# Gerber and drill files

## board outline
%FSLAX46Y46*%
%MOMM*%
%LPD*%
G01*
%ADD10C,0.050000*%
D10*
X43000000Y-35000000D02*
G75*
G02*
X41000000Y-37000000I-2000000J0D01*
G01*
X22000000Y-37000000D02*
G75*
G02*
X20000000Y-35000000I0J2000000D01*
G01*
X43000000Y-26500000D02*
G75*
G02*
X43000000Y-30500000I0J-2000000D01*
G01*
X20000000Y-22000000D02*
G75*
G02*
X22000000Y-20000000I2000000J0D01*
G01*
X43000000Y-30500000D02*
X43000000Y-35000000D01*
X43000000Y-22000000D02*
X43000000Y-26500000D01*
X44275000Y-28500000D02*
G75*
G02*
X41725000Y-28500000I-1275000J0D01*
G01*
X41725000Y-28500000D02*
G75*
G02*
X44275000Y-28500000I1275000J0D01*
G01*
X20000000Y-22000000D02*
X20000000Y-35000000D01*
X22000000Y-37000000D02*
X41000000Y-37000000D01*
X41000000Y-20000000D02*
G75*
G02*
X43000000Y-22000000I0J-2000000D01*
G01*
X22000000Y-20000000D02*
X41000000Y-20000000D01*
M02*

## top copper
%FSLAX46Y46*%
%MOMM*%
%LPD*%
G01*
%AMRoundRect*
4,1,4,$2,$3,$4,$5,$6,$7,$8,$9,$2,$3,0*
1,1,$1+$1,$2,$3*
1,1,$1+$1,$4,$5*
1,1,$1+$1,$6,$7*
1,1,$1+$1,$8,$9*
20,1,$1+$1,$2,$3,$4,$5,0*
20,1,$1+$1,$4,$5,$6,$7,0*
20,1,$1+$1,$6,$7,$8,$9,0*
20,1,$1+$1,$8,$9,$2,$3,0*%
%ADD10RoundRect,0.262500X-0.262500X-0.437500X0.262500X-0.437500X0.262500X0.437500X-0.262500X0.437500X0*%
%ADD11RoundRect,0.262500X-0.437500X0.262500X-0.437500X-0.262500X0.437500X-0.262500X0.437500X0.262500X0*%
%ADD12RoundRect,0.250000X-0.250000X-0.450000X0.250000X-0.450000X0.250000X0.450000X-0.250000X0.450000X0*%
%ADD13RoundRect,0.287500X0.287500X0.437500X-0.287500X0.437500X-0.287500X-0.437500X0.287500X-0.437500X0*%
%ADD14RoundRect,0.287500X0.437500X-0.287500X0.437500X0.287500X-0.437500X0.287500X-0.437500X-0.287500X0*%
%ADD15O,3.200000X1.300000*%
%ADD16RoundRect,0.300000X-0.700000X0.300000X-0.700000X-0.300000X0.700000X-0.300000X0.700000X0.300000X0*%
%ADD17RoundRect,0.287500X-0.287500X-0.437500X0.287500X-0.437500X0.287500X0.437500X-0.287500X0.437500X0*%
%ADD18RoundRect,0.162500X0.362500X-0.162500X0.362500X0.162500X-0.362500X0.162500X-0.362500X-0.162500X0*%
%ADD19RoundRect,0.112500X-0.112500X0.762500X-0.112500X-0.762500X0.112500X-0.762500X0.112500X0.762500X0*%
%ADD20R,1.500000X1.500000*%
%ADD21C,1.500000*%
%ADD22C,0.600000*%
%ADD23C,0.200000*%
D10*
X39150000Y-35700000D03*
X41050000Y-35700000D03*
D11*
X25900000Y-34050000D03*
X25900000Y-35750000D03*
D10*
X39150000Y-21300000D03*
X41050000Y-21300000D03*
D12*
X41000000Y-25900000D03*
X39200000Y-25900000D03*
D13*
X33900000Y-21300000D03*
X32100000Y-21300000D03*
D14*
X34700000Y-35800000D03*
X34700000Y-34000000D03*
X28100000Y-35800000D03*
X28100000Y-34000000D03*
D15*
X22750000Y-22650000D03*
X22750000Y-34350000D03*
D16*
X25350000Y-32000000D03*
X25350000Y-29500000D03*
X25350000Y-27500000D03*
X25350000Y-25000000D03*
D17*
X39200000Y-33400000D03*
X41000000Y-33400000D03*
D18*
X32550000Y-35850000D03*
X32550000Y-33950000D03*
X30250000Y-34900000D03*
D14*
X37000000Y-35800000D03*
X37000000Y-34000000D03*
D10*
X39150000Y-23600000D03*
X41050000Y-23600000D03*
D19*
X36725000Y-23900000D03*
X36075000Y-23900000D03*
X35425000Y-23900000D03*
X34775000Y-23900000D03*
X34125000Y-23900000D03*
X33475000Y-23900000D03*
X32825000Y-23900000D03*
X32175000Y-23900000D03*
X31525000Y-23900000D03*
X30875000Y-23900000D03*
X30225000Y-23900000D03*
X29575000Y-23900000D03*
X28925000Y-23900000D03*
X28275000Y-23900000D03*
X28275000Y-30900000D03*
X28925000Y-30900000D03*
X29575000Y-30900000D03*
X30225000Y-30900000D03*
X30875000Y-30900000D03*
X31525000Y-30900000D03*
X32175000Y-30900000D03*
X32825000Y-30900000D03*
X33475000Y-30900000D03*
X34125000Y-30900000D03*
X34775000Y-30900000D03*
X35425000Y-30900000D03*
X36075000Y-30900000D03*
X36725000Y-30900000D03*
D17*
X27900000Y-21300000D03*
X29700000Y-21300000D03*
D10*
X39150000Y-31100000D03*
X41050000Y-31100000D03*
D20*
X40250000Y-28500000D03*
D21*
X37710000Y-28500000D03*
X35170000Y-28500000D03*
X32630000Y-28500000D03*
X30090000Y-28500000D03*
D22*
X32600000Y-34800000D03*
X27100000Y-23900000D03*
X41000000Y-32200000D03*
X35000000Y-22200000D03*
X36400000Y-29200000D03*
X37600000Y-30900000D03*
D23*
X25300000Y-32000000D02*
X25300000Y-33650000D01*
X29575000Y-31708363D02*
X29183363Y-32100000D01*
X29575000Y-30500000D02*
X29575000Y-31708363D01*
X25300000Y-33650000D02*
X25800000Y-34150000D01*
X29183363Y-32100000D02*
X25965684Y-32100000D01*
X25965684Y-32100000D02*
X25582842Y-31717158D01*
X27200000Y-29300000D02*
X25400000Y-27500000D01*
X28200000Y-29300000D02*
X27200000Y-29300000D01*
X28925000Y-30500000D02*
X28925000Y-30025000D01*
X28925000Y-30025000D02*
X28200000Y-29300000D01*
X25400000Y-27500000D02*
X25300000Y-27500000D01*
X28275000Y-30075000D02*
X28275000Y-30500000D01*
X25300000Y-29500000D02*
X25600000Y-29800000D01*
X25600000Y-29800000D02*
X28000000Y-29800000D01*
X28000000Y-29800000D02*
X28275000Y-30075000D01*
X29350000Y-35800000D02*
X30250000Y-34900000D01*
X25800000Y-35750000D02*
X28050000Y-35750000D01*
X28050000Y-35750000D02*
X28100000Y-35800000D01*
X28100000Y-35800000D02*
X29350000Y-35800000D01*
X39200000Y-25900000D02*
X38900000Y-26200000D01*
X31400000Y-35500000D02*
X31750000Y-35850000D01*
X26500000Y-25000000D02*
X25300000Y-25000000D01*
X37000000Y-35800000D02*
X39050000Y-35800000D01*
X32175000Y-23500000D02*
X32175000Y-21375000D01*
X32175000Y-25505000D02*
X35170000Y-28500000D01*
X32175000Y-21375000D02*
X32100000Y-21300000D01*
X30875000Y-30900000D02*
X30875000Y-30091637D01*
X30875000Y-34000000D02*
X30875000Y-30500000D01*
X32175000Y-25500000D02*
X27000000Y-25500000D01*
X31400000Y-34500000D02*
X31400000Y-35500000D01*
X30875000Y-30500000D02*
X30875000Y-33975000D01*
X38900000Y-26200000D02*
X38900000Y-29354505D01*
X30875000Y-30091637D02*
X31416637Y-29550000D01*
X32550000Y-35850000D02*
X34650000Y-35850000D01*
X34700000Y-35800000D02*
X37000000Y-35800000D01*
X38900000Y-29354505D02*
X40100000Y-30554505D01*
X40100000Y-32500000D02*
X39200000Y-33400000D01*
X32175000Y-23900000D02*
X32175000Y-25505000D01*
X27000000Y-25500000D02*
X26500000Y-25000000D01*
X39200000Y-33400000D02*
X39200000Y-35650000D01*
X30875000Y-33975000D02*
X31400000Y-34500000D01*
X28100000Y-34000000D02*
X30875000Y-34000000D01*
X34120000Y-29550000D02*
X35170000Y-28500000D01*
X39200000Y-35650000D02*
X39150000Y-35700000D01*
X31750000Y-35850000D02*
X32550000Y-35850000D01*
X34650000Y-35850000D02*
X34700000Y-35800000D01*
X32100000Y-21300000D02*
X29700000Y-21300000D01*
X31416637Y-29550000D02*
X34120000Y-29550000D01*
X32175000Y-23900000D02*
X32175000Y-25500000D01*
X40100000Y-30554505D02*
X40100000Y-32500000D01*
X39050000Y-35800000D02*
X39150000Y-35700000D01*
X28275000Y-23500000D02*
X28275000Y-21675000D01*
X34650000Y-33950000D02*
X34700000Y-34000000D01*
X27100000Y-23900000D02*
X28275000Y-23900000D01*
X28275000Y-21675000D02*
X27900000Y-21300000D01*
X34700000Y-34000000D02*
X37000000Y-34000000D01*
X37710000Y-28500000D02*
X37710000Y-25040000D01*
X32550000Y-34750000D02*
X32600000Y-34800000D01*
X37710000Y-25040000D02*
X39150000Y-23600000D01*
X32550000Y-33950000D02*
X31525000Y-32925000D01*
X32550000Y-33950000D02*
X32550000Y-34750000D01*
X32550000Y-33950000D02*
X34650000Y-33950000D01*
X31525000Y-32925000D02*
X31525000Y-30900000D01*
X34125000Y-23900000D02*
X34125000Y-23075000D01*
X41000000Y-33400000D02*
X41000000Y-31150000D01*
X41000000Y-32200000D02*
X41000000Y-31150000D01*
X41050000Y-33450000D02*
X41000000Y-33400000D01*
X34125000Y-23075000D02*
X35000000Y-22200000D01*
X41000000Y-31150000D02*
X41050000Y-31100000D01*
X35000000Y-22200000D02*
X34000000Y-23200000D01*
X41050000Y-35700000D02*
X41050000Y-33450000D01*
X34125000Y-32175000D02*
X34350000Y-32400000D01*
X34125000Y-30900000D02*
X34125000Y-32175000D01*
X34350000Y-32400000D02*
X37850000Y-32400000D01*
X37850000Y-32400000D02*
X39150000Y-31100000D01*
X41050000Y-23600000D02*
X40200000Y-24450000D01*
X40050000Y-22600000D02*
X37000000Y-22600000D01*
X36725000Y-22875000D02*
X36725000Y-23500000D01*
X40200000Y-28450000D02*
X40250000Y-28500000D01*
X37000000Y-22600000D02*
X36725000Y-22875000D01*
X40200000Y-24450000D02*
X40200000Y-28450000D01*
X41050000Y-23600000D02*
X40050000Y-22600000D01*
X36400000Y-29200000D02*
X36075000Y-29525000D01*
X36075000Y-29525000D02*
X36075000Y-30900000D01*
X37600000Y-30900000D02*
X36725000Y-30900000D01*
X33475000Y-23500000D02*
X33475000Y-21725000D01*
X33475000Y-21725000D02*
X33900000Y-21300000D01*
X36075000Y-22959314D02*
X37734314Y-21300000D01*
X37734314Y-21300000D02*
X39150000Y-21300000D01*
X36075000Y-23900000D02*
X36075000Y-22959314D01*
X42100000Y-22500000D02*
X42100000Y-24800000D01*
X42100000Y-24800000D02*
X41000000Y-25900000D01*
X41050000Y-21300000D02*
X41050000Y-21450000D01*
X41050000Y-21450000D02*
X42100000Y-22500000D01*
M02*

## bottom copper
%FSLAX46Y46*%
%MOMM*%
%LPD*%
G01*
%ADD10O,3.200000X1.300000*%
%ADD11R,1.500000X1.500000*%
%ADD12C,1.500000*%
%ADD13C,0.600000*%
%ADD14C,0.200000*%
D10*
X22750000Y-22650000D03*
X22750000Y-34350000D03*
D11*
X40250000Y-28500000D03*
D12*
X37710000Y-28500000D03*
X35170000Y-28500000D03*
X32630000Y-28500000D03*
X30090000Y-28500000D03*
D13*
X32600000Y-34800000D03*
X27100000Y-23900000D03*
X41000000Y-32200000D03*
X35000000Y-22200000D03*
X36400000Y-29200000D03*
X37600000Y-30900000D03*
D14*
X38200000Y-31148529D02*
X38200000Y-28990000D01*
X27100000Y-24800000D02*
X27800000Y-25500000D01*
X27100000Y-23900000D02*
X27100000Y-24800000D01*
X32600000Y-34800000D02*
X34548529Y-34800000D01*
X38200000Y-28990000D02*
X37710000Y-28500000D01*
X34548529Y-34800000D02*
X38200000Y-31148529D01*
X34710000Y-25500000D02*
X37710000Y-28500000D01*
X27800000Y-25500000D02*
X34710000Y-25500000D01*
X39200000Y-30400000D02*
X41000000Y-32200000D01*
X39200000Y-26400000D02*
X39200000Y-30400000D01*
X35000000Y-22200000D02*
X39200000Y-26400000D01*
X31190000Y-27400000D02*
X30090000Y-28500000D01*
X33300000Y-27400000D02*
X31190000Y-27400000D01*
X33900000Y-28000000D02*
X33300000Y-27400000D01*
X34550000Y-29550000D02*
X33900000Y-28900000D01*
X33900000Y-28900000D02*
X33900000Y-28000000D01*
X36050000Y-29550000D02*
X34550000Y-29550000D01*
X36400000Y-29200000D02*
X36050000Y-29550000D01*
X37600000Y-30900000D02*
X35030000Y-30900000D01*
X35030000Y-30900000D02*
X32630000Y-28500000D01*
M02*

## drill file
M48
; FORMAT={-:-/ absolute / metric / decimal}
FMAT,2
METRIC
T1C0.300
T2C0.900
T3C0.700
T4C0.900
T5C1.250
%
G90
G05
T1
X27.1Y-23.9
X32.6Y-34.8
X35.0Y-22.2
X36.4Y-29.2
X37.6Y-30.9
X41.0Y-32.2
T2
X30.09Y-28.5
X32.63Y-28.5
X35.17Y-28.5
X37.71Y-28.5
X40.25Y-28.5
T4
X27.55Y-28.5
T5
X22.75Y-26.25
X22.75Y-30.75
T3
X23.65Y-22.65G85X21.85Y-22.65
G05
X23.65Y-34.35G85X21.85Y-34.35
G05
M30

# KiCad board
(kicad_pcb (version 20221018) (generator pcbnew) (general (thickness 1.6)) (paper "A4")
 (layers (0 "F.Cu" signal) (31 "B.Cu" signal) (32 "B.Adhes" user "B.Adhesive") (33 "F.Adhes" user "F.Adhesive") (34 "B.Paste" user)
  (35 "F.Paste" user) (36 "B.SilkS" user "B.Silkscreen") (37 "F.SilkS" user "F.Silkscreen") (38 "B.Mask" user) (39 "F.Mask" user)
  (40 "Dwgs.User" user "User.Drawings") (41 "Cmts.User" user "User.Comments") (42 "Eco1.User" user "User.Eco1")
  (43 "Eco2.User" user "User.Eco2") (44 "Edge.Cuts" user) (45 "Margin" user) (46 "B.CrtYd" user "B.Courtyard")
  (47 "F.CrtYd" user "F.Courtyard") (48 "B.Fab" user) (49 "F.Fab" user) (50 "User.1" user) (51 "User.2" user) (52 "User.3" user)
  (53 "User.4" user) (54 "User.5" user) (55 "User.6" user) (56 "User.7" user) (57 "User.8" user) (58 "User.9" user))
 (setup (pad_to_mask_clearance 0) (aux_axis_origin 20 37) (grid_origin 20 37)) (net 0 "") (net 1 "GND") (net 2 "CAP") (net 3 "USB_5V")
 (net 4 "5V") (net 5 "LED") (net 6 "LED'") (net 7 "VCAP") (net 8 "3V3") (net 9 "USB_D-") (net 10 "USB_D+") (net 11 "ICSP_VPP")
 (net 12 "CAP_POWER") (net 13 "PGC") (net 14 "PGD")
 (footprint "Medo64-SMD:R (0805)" (layer "F.Cu") (at 40.1 35.7)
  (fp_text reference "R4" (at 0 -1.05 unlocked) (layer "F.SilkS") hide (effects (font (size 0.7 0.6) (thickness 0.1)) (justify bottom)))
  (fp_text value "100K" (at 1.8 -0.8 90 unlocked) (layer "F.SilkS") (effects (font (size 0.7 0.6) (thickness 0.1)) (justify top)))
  (pad "1" smd roundrect (at -0.95 0) (size 1.05 1.4) (layers "F.Cu" "F.Paste" "F.Mask") (roundrect_rratio 0.25) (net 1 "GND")
   (thermal_bridge_angle 45))
  (pad "2" smd roundrect (at 0.95 0) (size 1.05 1.4) (layers "F.Cu" "F.Paste" "F.Mask") (roundrect_rratio 0.25) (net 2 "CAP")
   (thermal_bridge_angle 45)))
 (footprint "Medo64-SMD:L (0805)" (layer "F.Cu") (at 25.9 34.9 -90)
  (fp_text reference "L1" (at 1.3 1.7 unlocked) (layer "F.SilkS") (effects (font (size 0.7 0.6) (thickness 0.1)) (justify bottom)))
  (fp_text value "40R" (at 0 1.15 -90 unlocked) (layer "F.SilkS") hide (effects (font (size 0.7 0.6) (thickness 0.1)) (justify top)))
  (pad "1" smd roundrect (at -0.85 0 270) (size 1.05 1.4) (layers "F.Cu" "F.Paste" "F.Mask") (roundrect_rratio 0.25) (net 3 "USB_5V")
   (thermal_bridge_angle 45))
  (pad "2" smd roundrect (at 0.85 0 270) (size 1.05 1.4) (layers "F.Cu" "F.Paste" "F.Mask") (roundrect_rratio 0.25) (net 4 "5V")
   (thermal_bridge_angle 45)))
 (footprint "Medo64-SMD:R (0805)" (layer "F.Cu") (at 40.1 21.3)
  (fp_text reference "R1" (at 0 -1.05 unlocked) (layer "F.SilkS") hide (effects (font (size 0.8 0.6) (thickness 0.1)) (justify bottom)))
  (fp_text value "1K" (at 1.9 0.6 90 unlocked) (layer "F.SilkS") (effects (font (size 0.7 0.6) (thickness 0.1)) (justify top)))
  (pad "1" smd roundrect (at -0.95 0) (size 1.05 1.4) (layers "F.Cu" "F.Paste" "F.Mask") (roundrect_rratio 0.25) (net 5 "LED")
   (thermal_bridge_angle 45))
  (pad "2" smd roundrect (at 0.95 0) (size 1.05 1.4) (layers "F.Cu" "F.Paste" "F.Mask") (roundrect_rratio 0.25) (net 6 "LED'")
   (thermal_bridge_angle 45)))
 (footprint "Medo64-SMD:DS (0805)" (layer "F.Cu") (at 40.1 25.9)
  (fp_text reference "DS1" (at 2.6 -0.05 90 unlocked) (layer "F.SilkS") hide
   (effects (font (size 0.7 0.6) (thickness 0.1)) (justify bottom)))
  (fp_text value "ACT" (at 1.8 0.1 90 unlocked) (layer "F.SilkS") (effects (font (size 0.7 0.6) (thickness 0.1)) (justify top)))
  (pad "A" smd roundrect (at 0.9 0) (size 1 1.4) (layers "F.Cu" "F.Paste" "F.Mask") (roundrect_rratio 0.25) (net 6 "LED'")
   (thermal_bridge_angle 45))
  (pad "C" smd roundrect (at -0.9 0) (size 1 1.4) (layers "F.Cu" "F.Paste" "F.Mask") (roundrect_rratio 0.25) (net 1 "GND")
   (thermal_bridge_angle 45)))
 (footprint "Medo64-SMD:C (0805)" (layer "F.Cu") (at 33 21.3 180)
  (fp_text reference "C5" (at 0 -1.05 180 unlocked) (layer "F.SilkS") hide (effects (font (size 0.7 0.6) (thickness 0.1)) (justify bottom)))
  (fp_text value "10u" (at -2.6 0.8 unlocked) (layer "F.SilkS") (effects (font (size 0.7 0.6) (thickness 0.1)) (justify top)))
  (pad "1" smd roundrect (at -0.9 0 180) (size 1.15 1.45) (layers "F.Cu" "F.Paste" "F.Mask") (roundrect_rratio 0.25) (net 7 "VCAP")
   (thermal_bridge_angle 45))
  (pad "2" smd roundrect (at 0.9 0 180) (size 1.15 1.45) (layers "F.Cu" "F.Paste" "F.Mask") (roundrect_rratio 0.25) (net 1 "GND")
   (thermal_bridge_angle 45)))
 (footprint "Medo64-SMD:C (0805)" (layer "F.Cu") (at 34.7 34.9 90)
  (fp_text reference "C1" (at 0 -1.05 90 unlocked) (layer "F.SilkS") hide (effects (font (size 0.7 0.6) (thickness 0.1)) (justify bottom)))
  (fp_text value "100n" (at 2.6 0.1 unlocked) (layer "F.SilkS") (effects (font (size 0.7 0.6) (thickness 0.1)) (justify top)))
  (pad "1" smd roundrect (at -0.9 0 90) (size 1.15 1.45) (layers "F.Cu" "F.Paste" "F.Mask") (roundrect_rratio 0.25) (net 1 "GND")
   (thermal_bridge_angle 45))
  (pad "2" smd roundrect (at 0.9 0 90) (size 1.15 1.45) (layers "F.Cu" "F.Paste" "F.Mask") (roundrect_rratio 0.25) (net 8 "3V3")
   (thermal_bridge_angle 45)))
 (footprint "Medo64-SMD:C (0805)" (layer "F.Cu") (at 28.1 34.9 90)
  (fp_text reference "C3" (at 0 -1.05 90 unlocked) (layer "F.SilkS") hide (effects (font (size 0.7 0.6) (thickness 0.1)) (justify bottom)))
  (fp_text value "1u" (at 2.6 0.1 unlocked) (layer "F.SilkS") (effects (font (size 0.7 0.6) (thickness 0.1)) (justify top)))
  (pad "1" smd roundrect (at -0.9 0 90) (size 1.15 1.45) (layers "F.Cu" "F.Paste" "F.Mask") (roundrect_rratio 0.25) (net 4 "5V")
   (thermal_bridge_angle 45))
  (pad "2" smd roundrect (at 0.9 0 90) (size 1.15 1.45) (layers "F.Cu" "F.Paste" "F.Mask") (roundrect_rratio 0.25) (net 1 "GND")
   (thermal_bridge_angle 45)))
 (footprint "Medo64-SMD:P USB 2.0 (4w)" (layer "F.Cu") (at 22.75 28.5 -90)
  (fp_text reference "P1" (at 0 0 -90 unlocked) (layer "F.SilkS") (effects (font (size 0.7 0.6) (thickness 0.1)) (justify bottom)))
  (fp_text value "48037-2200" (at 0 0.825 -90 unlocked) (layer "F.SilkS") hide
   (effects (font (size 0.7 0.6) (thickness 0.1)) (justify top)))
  (pad "" np_thru_hole oval (at -5.85 0 270) (size 1.3 3.2) (drill oval 0.7 2.5) (layers "F&B.Cu" "*.Mask") (thermal_bridge_angle 45))
  (pad "" np_thru_hole circle (at -2.25 0 270) (size 1.25 1.25) (drill 1.25) (layers "F&B.Cu" "*.Mask"))
  (pad "" np_thru_hole circle (at 2.25 0 270) (size 1.25 1.25) (drill 1.25) (layers "F&B.Cu" "*.Mask"))
  (pad "" np_thru_hole oval (at 5.85 0 270) (size 1.3 3.2) (drill oval 0.7 2.5) (layers "F&B.Cu" "*.Mask") (thermal_bridge_angle 45))
  (pad "1" smd roundrect (at 3.5 -2.6 270) (size 1.2 2) (layers "F.Cu" "F.Paste" "F.Mask") (roundrect_rratio 0.25) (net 3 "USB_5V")
   (thermal_bridge_angle 45))
  (pad "2" smd roundrect (at 1 -2.6 270) (size 1.2 2) (layers "F.Cu" "F.Paste" "F.Mask") (roundrect_rratio 0.25) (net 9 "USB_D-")
   (thermal_bridge_angle 45))
  (pad "3" smd roundrect (at -1 -2.6 270) (size 1.2 2) (layers "F.Cu" "F.Paste" "F.Mask") (roundrect_rratio 0.25) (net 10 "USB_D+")
   (thermal_bridge_angle 45))
  (pad "4" smd roundrect (at -3.5 -2.6 270) (size 1.2 2) (layers "F.Cu" "F.Paste" "F.Mask") (roundrect_rratio 0.25) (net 1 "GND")
   (thermal_bridge_angle 45)))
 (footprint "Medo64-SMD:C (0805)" (layer "F.Cu") (at 40.1 33.4)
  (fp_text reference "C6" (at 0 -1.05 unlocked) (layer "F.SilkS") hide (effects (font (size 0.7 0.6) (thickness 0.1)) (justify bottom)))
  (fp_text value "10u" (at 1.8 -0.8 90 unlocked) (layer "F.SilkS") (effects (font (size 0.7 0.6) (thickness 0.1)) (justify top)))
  (pad "1" smd roundrect (at -0.9 0) (size 1.15 1.45) (layers "F.Cu" "F.Paste" "F.Mask") (roundrect_rratio 0.25) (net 1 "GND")
   (thermal_bridge_angle 45))
  (pad "2" smd roundrect (at 0.9 0) (size 1.15 1.45) (layers "F.Cu" "F.Paste" "F.Mask") (roundrect_rratio 0.25) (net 2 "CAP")
   (thermal_bridge_angle 45)))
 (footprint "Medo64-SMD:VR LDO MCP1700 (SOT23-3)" (layer "F.Cu") (at 31.4 34.9 90)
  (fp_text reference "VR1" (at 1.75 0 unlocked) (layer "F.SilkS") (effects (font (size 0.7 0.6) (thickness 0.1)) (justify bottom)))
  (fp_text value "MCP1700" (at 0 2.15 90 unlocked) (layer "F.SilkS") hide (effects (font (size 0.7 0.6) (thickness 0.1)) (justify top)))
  (pad "1" smd roundrect (at -0.95 1.15 90) (size 0.65 1.05) (layers "F.Cu" "F.Paste" "F.Mask") (roundrect_rratio 0.25) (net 1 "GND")
   (thermal_bridge_angle 45))
  (pad "2" smd roundrect (at 0.95 1.15 90) (size 0.65 1.05) (layers "F.Cu" "F.Paste" "F.Mask") (roundrect_rratio 0.25) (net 8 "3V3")
   (thermal_bridge_angle 45))
  (pad "3" smd roundrect (at 0 -1.15 90) (size 0.65 1.05) (layers "F.Cu" "F.Paste" "F.Mask") (roundrect_rratio 0.25) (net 4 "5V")
   (thermal_bridge_angle 45)))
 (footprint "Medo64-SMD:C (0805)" (layer "F.Cu") (at 37 34.9 90)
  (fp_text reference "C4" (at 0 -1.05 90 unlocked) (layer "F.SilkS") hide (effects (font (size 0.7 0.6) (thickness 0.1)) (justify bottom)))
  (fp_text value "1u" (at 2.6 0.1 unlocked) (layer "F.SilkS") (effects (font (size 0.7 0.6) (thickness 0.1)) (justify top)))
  (pad "1" smd roundrect (at -0.9 0 90) (size 1.15 1.45) (layers "F.Cu" "F.Paste" "F.Mask") (roundrect_rratio 0.25) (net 1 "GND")
   (thermal_bridge_angle 45))
  (pad "2" smd roundrect (at 0.9 0 90) (size 1.15 1.45) (layers "F.Cu" "F.Paste" "F.Mask") (roundrect_rratio 0.25) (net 8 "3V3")
   (thermal_bridge_angle 45)))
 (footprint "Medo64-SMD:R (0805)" (layer "F.Cu") (at 40.1 23.6)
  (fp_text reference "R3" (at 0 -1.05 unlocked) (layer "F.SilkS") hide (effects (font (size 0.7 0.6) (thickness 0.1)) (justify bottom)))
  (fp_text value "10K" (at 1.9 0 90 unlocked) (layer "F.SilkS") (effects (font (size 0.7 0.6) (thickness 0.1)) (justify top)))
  (pad "1" smd roundrect (at -0.95 0) (size 1.05 1.4) (layers "F.Cu" "F.Paste" "F.Mask") (roundrect_rratio 0.25) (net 8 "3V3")
   (thermal_bridge_angle 45))
  (pad "2" smd roundrect (at 0.95 0) (size 1.05 1.4) (layers "F.Cu" "F.Paste" "F.Mask") (roundrect_rratio 0.25) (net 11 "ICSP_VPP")
   (thermal_bridge_angle 45)))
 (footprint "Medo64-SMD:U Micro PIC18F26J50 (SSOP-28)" (layer "F.Cu") (at 32.5 27.4 -90)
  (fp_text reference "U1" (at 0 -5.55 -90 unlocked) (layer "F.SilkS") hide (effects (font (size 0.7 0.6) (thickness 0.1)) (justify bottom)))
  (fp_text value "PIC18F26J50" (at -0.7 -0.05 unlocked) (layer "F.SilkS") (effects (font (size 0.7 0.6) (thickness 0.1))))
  (pad "1" smd roundrect (at -3.5 -4.225 270) (size 1.75 0.45) (layers "F.Cu" "F.Paste" "F.Mask") (roundrect_rratio 0.25)
   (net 11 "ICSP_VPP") (thermal_bridge_angle 45))
  (pad "2" smd roundrect (at -3.5 -3.575 270) (size 1.75 0.45) (layers "F.Cu" "F.Paste" "F.Mask") (roundrect_rratio 0.25) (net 5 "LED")
   (thermal_bridge_angle 45))
  (pad "3" smd roundrect (at -3.5 -2.925 270) (size 1.75 0.45) (layers "F.Cu" "F.Paste" "F.Mask") (roundrect_rratio 0.25)
   (thermal_bridge_angle 45))
  (pad "4" smd roundrect (at -3.5 -2.275 270) (size 1.75 0.45) (layers "F.Cu" "F.Paste" "F.Mask") (roundrect_rratio 0.25)
   (thermal_bridge_angle 45))
  (pad "5" smd roundrect (at -3.5 -1.625 270) (size 1.75 0.45) (layers "F.Cu" "F.Paste" "F.Mask") (roundrect_rratio 0.25) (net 2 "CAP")
   (thermal_bridge_angle 45))
  (pad "6" smd roundrect (at -3.5 -0.975 270) (size 1.75 0.45) (layers "F.Cu" "F.Paste" "F.Mask") (roundrect_rratio 0.25) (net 7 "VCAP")
   (thermal_bridge_angle 45))
  (pad "7" smd roundrect (at -3.5 -0.325 270) (size 1.75 0.45) (layers "F.Cu" "F.Paste" "F.Mask") (roundrect_rratio 0.25)
   (thermal_bridge_angle 45))
  (pad "8" smd roundrect (at -3.5 0.325 270) (size 1.75 0.45) (layers "F.Cu" "F.Paste" "F.Mask") (roundrect_rratio 0.25) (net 1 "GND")
   (thermal_bridge_angle 45))
  (pad "9" smd roundrect (at -3.5 0.975 270) (size 1.75 0.45) (layers "F.Cu" "F.Paste" "F.Mask") (roundrect_rratio 0.25)
   (thermal_bridge_angle 45))
  (pad "10" smd roundrect (at -3.5 1.625 270) (size 1.75 0.45) (layers "F.Cu" "F.Paste" "F.Mask") (roundrect_rratio 0.25)
   (thermal_bridge_angle 45))
  (pad "11" smd roundrect (at -3.5 2.275 270) (size 1.75 0.45) (layers "F.Cu" "F.Paste" "F.Mask") (roundrect_rratio 0.25)
   (thermal_bridge_angle 45))
  (pad "12" smd roundrect (at -3.5 2.925 270) (size 1.75 0.45) (layers "F.Cu" "F.Paste" "F.Mask") (roundrect_rratio 0.25)
   (thermal_bridge_angle 45))
  (pad "13" smd roundrect (at -3.5 3.575 270) (size 1.75 0.45) (layers "F.Cu" "F.Paste" "F.Mask") (roundrect_rratio 0.25)
   (thermal_bridge_angle 45))
  (pad "14" smd roundrect (at -3.5 4.225 270) (size 1.75 0.45) (layers "F.Cu" "F.Paste" "F.Mask") (roundrect_rratio 0.25) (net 8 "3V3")
   (thermal_bridge_angle 45))
  (pad "15" smd roundrect (at 3.5 4.225 270) (size 1.75 0.45) (layers "F.Cu" "F.Paste" "F.Mask") (roundrect_rratio 0.25) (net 9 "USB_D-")
   (thermal_bridge_angle 45))
  (pad "16" smd roundrect (at 3.5 3.575 270) (size 1.75 0.45) (layers "F.Cu" "F.Paste" "F.Mask") (roundrect_rratio 0.25) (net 10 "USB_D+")
   (thermal_bridge_angle 45))
  (pad "17" smd roundrect (at 3.5 2.925 270) (size 1.75 0.45) (layers "F.Cu" "F.Paste" "F.Mask") (roundrect_rratio 0.25) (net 3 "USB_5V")
   (thermal_bridge_angle 45))
  (pad "18" smd roundrect (at 3.5 2.275 270) (size 1.75 0.45) (layers "F.Cu" "F.Paste" "F.Mask") (roundrect_rratio 0.25)
   (thermal_bridge_angle 45))
  (pad "19" smd roundrect (at 3.5 1.625 270) (size 1.75 0.45) (layers "F.Cu" "F.Paste" "F.Mask") (roundrect_rratio 0.25) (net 1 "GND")
   (thermal_bridge_angle 45))
  (pad "20" smd roundrect (at 3.5 0.975 270) (size 1.75 0.45) (layers "F.Cu" "F.Paste" "F.Mask") (roundrect_rratio 0.25) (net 8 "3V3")
   (thermal_bridge_angle 45))
  (pad "21" smd roundrect (at 3.5 0.325 270) (size 1.75 0.45) (layers "F.Cu" "F.Paste" "F.Mask") (roundrect_rratio 0.25)
   (thermal_bridge_angle 45))
  (pad "22" smd roundrect (at 3.5 -0.325 270) (size 1.75 0.45) (layers "F.Cu" "F.Paste" "F.Mask") (roundrect_rratio 0.25)
   (thermal_bridge_angle 45))
  (pad "23" smd roundrect (at 3.5 -0.975 270) (size 1.75 0.45) (layers "F.Cu" "F.Paste" "F.Mask") (roundrect_rratio 0.25)
   (thermal_bridge_angle 45))
  (pad "24" smd roundrect (at 3.5 -1.625 270) (size 1.75 0.45) (layers "F.Cu" "F.Paste" "F.Mask") (roundrect_rratio 0.25)
   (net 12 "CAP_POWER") (thermal_bridge_angle 45))
  (pad "25" smd roundrect (at 3.5 -2.275 270) (size 1.75 0.45) (layers "F.Cu" "F.Paste" "F.Mask") (roundrect_rratio 0.25)
   (thermal_bridge_angle 45))
  (pad "26" smd roundrect (at 3.5 -2.925 270) (size 1.75 0.45) (layers "F.Cu" "F.Paste" "F.Mask") (roundrect_rratio 0.25)
   (thermal_bridge_angle 45))
  (pad "27" smd roundrect (at 3.5 -3.575 270) (size 1.75 0.45) (layers "F.Cu" "F.Paste" "F.Mask") (roundrect_rratio 0.25) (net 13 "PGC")
   (thermal_bridge_angle 45))
  (pad "28" smd roundrect (at 3.5 -4.225 270) (size 1.75 0.45) (layers "F.Cu" "F.Paste" "F.Mask") (roundrect_rratio 0.25) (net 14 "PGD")
   (thermal_bridge_angle 45)))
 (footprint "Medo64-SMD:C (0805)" (layer "F.Cu") (at 28.8 21.3)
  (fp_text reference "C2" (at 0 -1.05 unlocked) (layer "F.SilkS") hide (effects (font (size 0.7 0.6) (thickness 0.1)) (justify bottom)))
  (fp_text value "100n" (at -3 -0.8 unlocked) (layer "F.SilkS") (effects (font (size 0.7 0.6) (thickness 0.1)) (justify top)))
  (pad "1" smd roundrect (at -0.9 0) (size 1.15 1.45) (layers "F.Cu" "F.Paste" "F.Mask") (roundrect_rratio 0.25) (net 8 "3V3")
   (thermal_bridge_angle 45))
  (pad "2" smd roundrect (at 0.9 0) (size 1.15 1.45) (layers "F.Cu" "F.Paste" "F.Mask") (roundrect_rratio 0.25) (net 1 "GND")
   (thermal_bridge_angle 45)))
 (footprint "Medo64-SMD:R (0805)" (layer "F.Cu") (at 40.1 31.1)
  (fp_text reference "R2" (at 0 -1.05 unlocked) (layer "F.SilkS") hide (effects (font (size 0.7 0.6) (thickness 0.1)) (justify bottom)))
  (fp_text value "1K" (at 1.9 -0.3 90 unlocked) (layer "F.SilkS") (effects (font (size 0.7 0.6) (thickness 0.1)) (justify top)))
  (pad "1" smd roundrect (at -0.95 0) (size 1.05 1.4) (layers "F.Cu" "F.Paste" "F.Mask") (roundrect_rratio 0.25) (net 12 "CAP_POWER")
   (thermal_bridge_angle 45))
  (pad "2" smd roundrect (at 0.95 0) (size 1.05 1.4) (layers "F.Cu" "F.Paste" "F.Mask") (roundrect_rratio 0.25) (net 2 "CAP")
   (thermal_bridge_angle 45)))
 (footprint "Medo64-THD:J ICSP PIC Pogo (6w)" (layer "B.Cu") (at 33.9 28.5 180)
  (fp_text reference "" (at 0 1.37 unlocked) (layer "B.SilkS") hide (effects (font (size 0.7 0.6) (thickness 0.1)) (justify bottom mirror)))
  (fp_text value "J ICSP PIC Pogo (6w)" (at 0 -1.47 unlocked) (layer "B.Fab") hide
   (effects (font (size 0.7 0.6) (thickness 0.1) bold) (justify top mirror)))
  (pad "" np_thru_hole circle (at 6.35 0 180) (size 0.9 0.9) (drill 0.9) (layers "F&B.Cu" "*.Mask"))
  (pad "1" thru_hole rect (at -6.35 0 180) (size 1.5 1.5) (drill 0.9) (layers "*.Cu" "*.Mask") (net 11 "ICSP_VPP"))
  (pad "2" thru_hole circle (at -3.81 0 180) (size 1.5 1.5) (drill 0.9) (layers "*.Cu" "*.Mask") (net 8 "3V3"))
  (pad "3" thru_hole circle (at -1.27 0 180) (size 1.5 1.5) (drill 0.9) (layers "*.Cu" "*.Mask") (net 1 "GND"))
  (pad "4" thru_hole circle (at 1.27 0 180) (size 1.5 1.5) (drill 0.9) (layers "*.Cu" "*.Mask") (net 14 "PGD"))
  (pad "5" thru_hole circle (at 3.81 0 180) (size 1.5 1.5) (drill 0.9) (layers "*.Cu" "*.Mask") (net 13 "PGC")))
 (gr_arc (start 43 35) (mid 42.414214 36.414214) (end 41 37) (stroke (width 0.05) (type default)) (layer "Edge.Cuts"))
 (gr_arc (start 22 37) (mid 20.585786 36.414214) (end 20 35) (stroke (width 0.05) (type default)) (layer "Edge.Cuts"))
 (gr_arc (start 43 26.5) (mid 45 28.5) (end 43 30.5) (stroke (width 0.05) (type default)) (layer "Edge.Cuts"))
 (gr_arc (start 20 22) (mid 20.585786 20.585786) (end 22 20) (stroke (width 0.05) (type default)) (layer "Edge.Cuts"))
 (gr_line (start 43 30.5) (end 43 35) (stroke (width 0.05) (type default)) (layer "Edge.Cuts"))
 (gr_line (start 43 22) (end 43 26.5) (stroke (width 0.05) (type default)) (layer "Edge.Cuts"))
 (gr_circle (center 43 28.5) (end 44.275 28.5) (stroke (width 0.05) (type default)) (fill none) (layer "Edge.Cuts"))
 (gr_line (start 20 22) (end 20 35) (stroke (width 0.05) (type default)) (layer "Edge.Cuts"))
 (gr_line (start 22 37) (end 41 37) (stroke (width 0.05) (type default)) (layer "Edge.Cuts"))
 (gr_arc (start 41 20) (mid 42.414214 20.585786) (end 43 22) (stroke (width 0.05) (type default)) (layer "Edge.Cuts"))
 (gr_line (start 22 20) (end 41 20) (stroke (width 0.05) (type default)) (layer "Edge.Cuts"))
 (segment (start 25.3 32) (end 25.3 33.65) (width 0.2) (layer "F.Cu") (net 3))
 (segment (start 29.575 31.708363) (end 29.183363 32.1) (width 0.2) (layer "F.Cu") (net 3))
 (segment (start 29.575 30.5) (end 29.575 31.708363) (width 0.2) (layer "F.Cu") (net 3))
 (segment (start 25.3 33.65) (end 25.8 34.15) (width 0.2) (layer "F.Cu") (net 3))
 (segment (start 29.183363 32.1) (end 25.965684 32.1) (width 0.2) (layer "F.Cu") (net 3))
 (segment (start 25.965684 32.1) (end 25.582842 31.717158) (width 0.2) (layer "F.Cu") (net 3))
 (segment (start 27.2 29.3) (end 25.4 27.5) (width 0.2) (layer "F.Cu") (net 10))
 (segment (start 28.2 29.3) (end 27.2 29.3) (width 0.2) (layer "F.Cu") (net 10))
 (segment (start 28.925 30.5) (end 28.925 30.025) (width 0.2) (layer "F.Cu") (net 10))
 (segment (start 28.925 30.025) (end 28.2 29.3) (width 0.2) (layer "F.Cu") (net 10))
 (segment (start 25.4 27.5) (end 25.3 27.5) (width 0.2) (layer "F.Cu") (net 10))
 (segment (start 28.275 30.075) (end 28.275 30.5) (width 0.2) (layer "F.Cu") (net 9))
 (segment (start 25.3 29.5) (end 25.6 29.8) (width 0.2) (layer "F.Cu") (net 9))
 (segment (start 25.6 29.8) (end 28 29.8) (width 0.2) (layer "F.Cu") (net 9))
 (segment (start 28 29.8) (end 28.275 30.075) (width 0.2) (layer "F.Cu") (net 9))
 (segment (start 29.35 35.8) (end 30.25 34.9) (width 0.2) (layer "F.Cu") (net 4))
 (segment (start 25.8 35.75) (end 28.05 35.75) (width 0.2) (layer "F.Cu") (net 4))
 (segment (start 28.05 35.75) (end 28.1 35.8) (width 0.2) (layer "F.Cu") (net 4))
 (segment (start 28.1 35.8) (end 29.35 35.8) (width 0.2) (layer "F.Cu") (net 4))
 (segment (start 39.2 25.9) (end 38.9 26.2) (width 0.2) (layer "F.Cu") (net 1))
 (segment (start 31.4 35.5) (end 31.75 35.85) (width 0.2) (layer "F.Cu") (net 1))
 (segment (start 26.5 25) (end 25.3 25) (width 0.2) (layer "F.Cu") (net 1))
 (segment (start 37 35.8) (end 39.05 35.8) (width 0.2) (layer "F.Cu") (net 1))
 (segment (start 32.175 23.5) (end 32.175 21.375) (width 0.2) (layer "F.Cu") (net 1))
 (segment (start 32.175 25.505) (end 35.17 28.5) (width 0.2) (layer "F.Cu") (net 1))
 (segment (start 32.175 21.375) (end 32.1 21.3) (width 0.2) (layer "F.Cu") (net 1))
 (segment (start 30.875 30.9) (end 30.875 30.091637) (width 0.2) (layer "F.Cu") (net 1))
 (segment (start 30.875 34) (end 30.875 30.5) (width 0.2) (layer "F.Cu") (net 1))
 (segment (start 32.175 25.5) (end 27 25.5) (width 0.2) (layer "F.Cu") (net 1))
 (segment (start 31.4 34.5) (end 31.4 35.5) (width 0.2) (layer "F.Cu") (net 1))
 (segment (start 30.875 30.5) (end 30.875 33.975) (width 0.2) (layer "F.Cu") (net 1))
 (segment (start 38.9 26.2) (end 38.9 29.354505) (width 0.2) (layer "F.Cu") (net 1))
 (segment (start 30.875 30.091637) (end 31.416637 29.55) (width 0.2) (layer "F.Cu") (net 1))
 (segment (start 32.55 35.85) (end 34.65 35.85) (width 0.2) (layer "F.Cu") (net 1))
 (segment (start 34.7 35.8) (end 37 35.8) (width 0.2) (layer "F.Cu") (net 1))
 (segment (start 38.9 29.354505) (end 40.1 30.554505) (width 0.2) (layer "F.Cu") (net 1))
 (segment (start 40.1 32.5) (end 39.2 33.4) (width 0.2) (layer "F.Cu") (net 1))
 (segment (start 32.175 23.9) (end 32.175 25.505) (width 0.2) (layer "F.Cu") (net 1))
 (segment (start 27 25.5) (end 26.5 25) (width 0.2) (layer "F.Cu") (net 1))
 (segment (start 39.2 33.4) (end 39.2 35.65) (width 0.2) (layer "F.Cu") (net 1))
 (segment (start 30.875 33.975) (end 31.4 34.5) (width 0.2) (layer "F.Cu") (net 1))
 (segment (start 28.1 34) (end 30.875 34) (width 0.2) (layer "F.Cu") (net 1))
 (segment (start 34.12 29.55) (end 35.17 28.5) (width 0.2) (layer "F.Cu") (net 1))
 (segment (start 39.2 35.65) (end 39.15 35.7) (width 0.2) (layer "F.Cu") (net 1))
 (segment (start 31.75 35.85) (end 32.55 35.85) (width 0.2) (layer "F.Cu") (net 1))
 (segment (start 34.65 35.85) (end 34.7 35.8) (width 0.2) (layer "F.Cu") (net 1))
 (segment (start 32.1 21.3) (end 29.7 21.3) (width 0.2) (layer "F.Cu") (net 1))
 (segment (start 31.416637 29.55) (end 34.12 29.55) (width 0.2) (layer "F.Cu") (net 1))
 (segment (start 32.175 23.9) (end 32.175 25.5) (width 0.2) (layer "F.Cu") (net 1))
 (segment (start 40.1 30.554505) (end 40.1 32.5) (width 0.2) (layer "F.Cu") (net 1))
 (segment (start 39.05 35.8) (end 39.15 35.7) (width 0.2) (layer "F.Cu") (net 1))
 (segment (start 28.275 23.5) (end 28.275 21.675) (width 0.2) (layer "F.Cu") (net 8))
 (segment (start 34.65 33.95) (end 34.7 34) (width 0.2) (layer "F.Cu") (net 8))
 (segment (start 27.1 23.9) (end 28.275 23.9) (width 0.2) (layer "F.Cu") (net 8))
 (segment (start 28.275 21.675) (end 27.9 21.3) (width 0.2) (layer "F.Cu") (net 8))
 (segment (start 34.7 34) (end 37 34) (width 0.2) (layer "F.Cu") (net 8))
 (segment (start 37.71 28.5) (end 37.71 25.04) (width 0.2) (layer "F.Cu") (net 8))
 (segment (start 32.55 34.75) (end 32.6 34.8) (width 0.2) (layer "F.Cu") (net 8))
 (segment (start 37.71 25.04) (end 39.15 23.6) (width 0.2) (layer "F.Cu") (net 8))
 (segment (start 32.55 33.95) (end 31.525 32.925) (width 0.2) (layer "F.Cu") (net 8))
 (segment (start 32.55 33.95) (end 32.55 34.75) (width 0.2) (layer "F.Cu") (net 8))
 (segment (start 32.55 33.95) (end 34.65 33.95) (width 0.2) (layer "F.Cu") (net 8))
 (segment (start 31.525 32.925) (end 31.525 30.9) (width 0.2) (layer "F.Cu") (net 8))
 (via (at 32.6 34.8) (size 0.6) (drill 0.3) (layers "F.Cu" "B.Cu") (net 8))
 (via (at 27.1 23.9) (size 0.6) (drill 0.3) (layers "F.Cu" "B.Cu") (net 8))
 (segment (start 38.2 31.148529) (end 38.2 28.99) (width 0.2) (layer "B.Cu") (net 8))
 (segment (start 27.1 24.8) (end 27.8 25.5) (width 0.2) (layer "B.Cu") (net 8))
 (segment (start 27.1 23.9) (end 27.1 24.8) (width 0.2) (layer "B.Cu") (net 8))
 (segment (start 32.6 34.8) (end 34.548529 34.8) (width 0.2) (layer "B.Cu") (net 8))
 (segment (start 38.2 28.99) (end 37.71 28.5) (width 0.2) (layer "B.Cu") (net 8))
 (segment (start 34.548529 34.8) (end 38.2 31.148529) (width 0.2) (layer "B.Cu") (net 8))
 (segment (start 34.71 25.5) (end 37.71 28.5) (width 0.2) (layer "B.Cu") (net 8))
 (segment (start 27.8 25.5) (end 34.71 25.5) (width 0.2) (layer "B.Cu") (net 8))
 (segment (start 34.125 23.9) (end 34.125 23.075) (width 0.2) (layer "F.Cu") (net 2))
 (segment (start 41 33.4) (end 41 31.15) (width 0.2) (layer "F.Cu") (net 2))
 (segment (start 41 32.2) (end 41 31.15) (width 0.2) (layer "F.Cu") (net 2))
 (segment (start 41.05 33.45) (end 41 33.4) (width 0.2) (layer "F.Cu") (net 2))
 (segment (start 34.125 23.075) (end 35 22.2) (width 0.2) (layer "F.Cu") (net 2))
 (segment (start 41 31.15) (end 41.05 31.1) (width 0.2) (layer "F.Cu") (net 2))
 (segment (start 35 22.2) (end 34 23.2) (width 0.2) (layer "F.Cu") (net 2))
 (segment (start 41.05 35.7) (end 41.05 33.45) (width 0.2) (layer "F.Cu") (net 2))
 (via (at 41 32.2) (size 0.6) (drill 0.3) (layers "F.Cu" "B.Cu") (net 2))
 (via (at 35 22.2) (size 0.6) (drill 0.3) (layers "F.Cu" "B.Cu") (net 2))
 (segment (start 39.2 30.4) (end 41 32.2) (width 0.2) (layer "B.Cu") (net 2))
 (segment (start 39.2 26.4) (end 39.2 30.4) (width 0.2) (layer "B.Cu") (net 2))
 (segment (start 35 22.2) (end 39.2 26.4) (width 0.2) (layer "B.Cu") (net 2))
 (segment (start 34.125 32.175) (end 34.35 32.4) (width 0.2) (layer "F.Cu") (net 12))
 (segment (start 34.125 30.9) (end 34.125 32.175) (width 0.2) (layer "F.Cu") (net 12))
 (segment (start 34.35 32.4) (end 37.85 32.4) (width 0.2) (layer "F.Cu") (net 12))
 (segment (start 37.85 32.4) (end 39.15 31.1) (width 0.2) (layer "F.Cu") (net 12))
 (segment (start 41.05 23.6) (end 40.2 24.45) (width 0.2) (layer "F.Cu") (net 11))
 (segment (start 40.05 22.6) (end 37 22.6) (width 0.2) (layer "F.Cu") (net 11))
 (segment (start 36.725 22.875) (end 36.725 23.5) (width 0.2) (layer "F.Cu") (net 11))
 (segment (start 40.2 28.45) (end 40.25 28.5) (width 0.2) (layer "F.Cu") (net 11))
 (segment (start 37 22.6) (end 36.725 22.875) (width 0.2) (layer "F.Cu") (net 11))
 (segment (start 40.2 24.45) (end 40.2 28.45) (width 0.2) (layer "F.Cu") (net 11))
 (segment (start 41.05 23.6) (end 40.05 22.6) (width 0.2) (layer "F.Cu") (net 11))
 (segment (start 36.4 29.2) (end 36.075 29.525) (width 0.2) (layer "F.Cu") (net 13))
 (segment (start 36.075 29.525) (end 36.075 30.9) (width 0.2) (layer "F.Cu") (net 13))
 (via (at 36.4 29.2) (size 0.6) (drill 0.3) (layers "F.Cu" "B.Cu") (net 13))
 (segment (start 31.19 27.4) (end 30.09 28.5) (width 0.2) (layer "B.Cu") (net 13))
 (segment (start 33.3 27.4) (end 31.19 27.4) (width 0.2) (layer "B.Cu") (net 13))
 (segment (start 33.9 28) (end 33.3 27.4) (width 0.2) (layer "B.Cu") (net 13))
 (segment (start 34.55 29.55) (end 33.9 28.9) (width 0.2) (layer "B.Cu") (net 13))
 (segment (start 33.9 28.9) (end 33.9 28) (width 0.2) (layer "B.Cu") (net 13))
 (segment (start 36.05 29.55) (end 34.55 29.55) (width 0.2) (layer "B.Cu") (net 13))
 (segment (start 36.4 29.2) (end 36.05 29.55) (width 0.2) (layer "B.Cu") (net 13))
 (segment (start 37.6 30.9) (end 36.725 30.9) (width 0.2) (layer "F.Cu") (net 14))
 (via (at 37.6 30.9) (size 0.6) (drill 0.3) (layers "F.Cu" "B.Cu") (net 14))
 (segment (start 37.6 30.9) (end 35.03 30.9) (width 0.2) (layer "B.Cu") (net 14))
 (segment (start 35.03 30.9) (end 32.63 28.5) (width 0.2) (layer "B.Cu") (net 14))
 (segment (start 33.475 23.5) (end 33.475 21.725) (width 0.2) (layer "F.Cu") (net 7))
 (segment (start 33.475 21.725) (end 33.9 21.3) (width 0.2) (layer "F.Cu") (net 7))
 (segment (start 36.075 22.959314) (end 37.734314 21.3) (width 0.2) (layer "F.Cu") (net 5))
 (segment (start 37.734314 21.3) (end 39.15 21.3) (width 0.2) (layer "F.Cu") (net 5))
 (segment (start 36.075 23.9) (end 36.075 22.959314) (width 0.2) (layer "F.Cu") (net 5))
 (segment (start 42.1 22.5) (end 42.1 24.8) (width 0.2) (layer "F.Cu") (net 6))
 (segment (start 42.1 24.8) (end 41 25.9) (width 0.2) (layer "F.Cu") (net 6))
 (segment (start 41.05 21.3) (end 41.05 21.45) (width 0.2) (layer "F.Cu") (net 6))
 (segment (start 41.05 21.45) (end 42.1 22.5) (width 0.2) (layer "F.Cu") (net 6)))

